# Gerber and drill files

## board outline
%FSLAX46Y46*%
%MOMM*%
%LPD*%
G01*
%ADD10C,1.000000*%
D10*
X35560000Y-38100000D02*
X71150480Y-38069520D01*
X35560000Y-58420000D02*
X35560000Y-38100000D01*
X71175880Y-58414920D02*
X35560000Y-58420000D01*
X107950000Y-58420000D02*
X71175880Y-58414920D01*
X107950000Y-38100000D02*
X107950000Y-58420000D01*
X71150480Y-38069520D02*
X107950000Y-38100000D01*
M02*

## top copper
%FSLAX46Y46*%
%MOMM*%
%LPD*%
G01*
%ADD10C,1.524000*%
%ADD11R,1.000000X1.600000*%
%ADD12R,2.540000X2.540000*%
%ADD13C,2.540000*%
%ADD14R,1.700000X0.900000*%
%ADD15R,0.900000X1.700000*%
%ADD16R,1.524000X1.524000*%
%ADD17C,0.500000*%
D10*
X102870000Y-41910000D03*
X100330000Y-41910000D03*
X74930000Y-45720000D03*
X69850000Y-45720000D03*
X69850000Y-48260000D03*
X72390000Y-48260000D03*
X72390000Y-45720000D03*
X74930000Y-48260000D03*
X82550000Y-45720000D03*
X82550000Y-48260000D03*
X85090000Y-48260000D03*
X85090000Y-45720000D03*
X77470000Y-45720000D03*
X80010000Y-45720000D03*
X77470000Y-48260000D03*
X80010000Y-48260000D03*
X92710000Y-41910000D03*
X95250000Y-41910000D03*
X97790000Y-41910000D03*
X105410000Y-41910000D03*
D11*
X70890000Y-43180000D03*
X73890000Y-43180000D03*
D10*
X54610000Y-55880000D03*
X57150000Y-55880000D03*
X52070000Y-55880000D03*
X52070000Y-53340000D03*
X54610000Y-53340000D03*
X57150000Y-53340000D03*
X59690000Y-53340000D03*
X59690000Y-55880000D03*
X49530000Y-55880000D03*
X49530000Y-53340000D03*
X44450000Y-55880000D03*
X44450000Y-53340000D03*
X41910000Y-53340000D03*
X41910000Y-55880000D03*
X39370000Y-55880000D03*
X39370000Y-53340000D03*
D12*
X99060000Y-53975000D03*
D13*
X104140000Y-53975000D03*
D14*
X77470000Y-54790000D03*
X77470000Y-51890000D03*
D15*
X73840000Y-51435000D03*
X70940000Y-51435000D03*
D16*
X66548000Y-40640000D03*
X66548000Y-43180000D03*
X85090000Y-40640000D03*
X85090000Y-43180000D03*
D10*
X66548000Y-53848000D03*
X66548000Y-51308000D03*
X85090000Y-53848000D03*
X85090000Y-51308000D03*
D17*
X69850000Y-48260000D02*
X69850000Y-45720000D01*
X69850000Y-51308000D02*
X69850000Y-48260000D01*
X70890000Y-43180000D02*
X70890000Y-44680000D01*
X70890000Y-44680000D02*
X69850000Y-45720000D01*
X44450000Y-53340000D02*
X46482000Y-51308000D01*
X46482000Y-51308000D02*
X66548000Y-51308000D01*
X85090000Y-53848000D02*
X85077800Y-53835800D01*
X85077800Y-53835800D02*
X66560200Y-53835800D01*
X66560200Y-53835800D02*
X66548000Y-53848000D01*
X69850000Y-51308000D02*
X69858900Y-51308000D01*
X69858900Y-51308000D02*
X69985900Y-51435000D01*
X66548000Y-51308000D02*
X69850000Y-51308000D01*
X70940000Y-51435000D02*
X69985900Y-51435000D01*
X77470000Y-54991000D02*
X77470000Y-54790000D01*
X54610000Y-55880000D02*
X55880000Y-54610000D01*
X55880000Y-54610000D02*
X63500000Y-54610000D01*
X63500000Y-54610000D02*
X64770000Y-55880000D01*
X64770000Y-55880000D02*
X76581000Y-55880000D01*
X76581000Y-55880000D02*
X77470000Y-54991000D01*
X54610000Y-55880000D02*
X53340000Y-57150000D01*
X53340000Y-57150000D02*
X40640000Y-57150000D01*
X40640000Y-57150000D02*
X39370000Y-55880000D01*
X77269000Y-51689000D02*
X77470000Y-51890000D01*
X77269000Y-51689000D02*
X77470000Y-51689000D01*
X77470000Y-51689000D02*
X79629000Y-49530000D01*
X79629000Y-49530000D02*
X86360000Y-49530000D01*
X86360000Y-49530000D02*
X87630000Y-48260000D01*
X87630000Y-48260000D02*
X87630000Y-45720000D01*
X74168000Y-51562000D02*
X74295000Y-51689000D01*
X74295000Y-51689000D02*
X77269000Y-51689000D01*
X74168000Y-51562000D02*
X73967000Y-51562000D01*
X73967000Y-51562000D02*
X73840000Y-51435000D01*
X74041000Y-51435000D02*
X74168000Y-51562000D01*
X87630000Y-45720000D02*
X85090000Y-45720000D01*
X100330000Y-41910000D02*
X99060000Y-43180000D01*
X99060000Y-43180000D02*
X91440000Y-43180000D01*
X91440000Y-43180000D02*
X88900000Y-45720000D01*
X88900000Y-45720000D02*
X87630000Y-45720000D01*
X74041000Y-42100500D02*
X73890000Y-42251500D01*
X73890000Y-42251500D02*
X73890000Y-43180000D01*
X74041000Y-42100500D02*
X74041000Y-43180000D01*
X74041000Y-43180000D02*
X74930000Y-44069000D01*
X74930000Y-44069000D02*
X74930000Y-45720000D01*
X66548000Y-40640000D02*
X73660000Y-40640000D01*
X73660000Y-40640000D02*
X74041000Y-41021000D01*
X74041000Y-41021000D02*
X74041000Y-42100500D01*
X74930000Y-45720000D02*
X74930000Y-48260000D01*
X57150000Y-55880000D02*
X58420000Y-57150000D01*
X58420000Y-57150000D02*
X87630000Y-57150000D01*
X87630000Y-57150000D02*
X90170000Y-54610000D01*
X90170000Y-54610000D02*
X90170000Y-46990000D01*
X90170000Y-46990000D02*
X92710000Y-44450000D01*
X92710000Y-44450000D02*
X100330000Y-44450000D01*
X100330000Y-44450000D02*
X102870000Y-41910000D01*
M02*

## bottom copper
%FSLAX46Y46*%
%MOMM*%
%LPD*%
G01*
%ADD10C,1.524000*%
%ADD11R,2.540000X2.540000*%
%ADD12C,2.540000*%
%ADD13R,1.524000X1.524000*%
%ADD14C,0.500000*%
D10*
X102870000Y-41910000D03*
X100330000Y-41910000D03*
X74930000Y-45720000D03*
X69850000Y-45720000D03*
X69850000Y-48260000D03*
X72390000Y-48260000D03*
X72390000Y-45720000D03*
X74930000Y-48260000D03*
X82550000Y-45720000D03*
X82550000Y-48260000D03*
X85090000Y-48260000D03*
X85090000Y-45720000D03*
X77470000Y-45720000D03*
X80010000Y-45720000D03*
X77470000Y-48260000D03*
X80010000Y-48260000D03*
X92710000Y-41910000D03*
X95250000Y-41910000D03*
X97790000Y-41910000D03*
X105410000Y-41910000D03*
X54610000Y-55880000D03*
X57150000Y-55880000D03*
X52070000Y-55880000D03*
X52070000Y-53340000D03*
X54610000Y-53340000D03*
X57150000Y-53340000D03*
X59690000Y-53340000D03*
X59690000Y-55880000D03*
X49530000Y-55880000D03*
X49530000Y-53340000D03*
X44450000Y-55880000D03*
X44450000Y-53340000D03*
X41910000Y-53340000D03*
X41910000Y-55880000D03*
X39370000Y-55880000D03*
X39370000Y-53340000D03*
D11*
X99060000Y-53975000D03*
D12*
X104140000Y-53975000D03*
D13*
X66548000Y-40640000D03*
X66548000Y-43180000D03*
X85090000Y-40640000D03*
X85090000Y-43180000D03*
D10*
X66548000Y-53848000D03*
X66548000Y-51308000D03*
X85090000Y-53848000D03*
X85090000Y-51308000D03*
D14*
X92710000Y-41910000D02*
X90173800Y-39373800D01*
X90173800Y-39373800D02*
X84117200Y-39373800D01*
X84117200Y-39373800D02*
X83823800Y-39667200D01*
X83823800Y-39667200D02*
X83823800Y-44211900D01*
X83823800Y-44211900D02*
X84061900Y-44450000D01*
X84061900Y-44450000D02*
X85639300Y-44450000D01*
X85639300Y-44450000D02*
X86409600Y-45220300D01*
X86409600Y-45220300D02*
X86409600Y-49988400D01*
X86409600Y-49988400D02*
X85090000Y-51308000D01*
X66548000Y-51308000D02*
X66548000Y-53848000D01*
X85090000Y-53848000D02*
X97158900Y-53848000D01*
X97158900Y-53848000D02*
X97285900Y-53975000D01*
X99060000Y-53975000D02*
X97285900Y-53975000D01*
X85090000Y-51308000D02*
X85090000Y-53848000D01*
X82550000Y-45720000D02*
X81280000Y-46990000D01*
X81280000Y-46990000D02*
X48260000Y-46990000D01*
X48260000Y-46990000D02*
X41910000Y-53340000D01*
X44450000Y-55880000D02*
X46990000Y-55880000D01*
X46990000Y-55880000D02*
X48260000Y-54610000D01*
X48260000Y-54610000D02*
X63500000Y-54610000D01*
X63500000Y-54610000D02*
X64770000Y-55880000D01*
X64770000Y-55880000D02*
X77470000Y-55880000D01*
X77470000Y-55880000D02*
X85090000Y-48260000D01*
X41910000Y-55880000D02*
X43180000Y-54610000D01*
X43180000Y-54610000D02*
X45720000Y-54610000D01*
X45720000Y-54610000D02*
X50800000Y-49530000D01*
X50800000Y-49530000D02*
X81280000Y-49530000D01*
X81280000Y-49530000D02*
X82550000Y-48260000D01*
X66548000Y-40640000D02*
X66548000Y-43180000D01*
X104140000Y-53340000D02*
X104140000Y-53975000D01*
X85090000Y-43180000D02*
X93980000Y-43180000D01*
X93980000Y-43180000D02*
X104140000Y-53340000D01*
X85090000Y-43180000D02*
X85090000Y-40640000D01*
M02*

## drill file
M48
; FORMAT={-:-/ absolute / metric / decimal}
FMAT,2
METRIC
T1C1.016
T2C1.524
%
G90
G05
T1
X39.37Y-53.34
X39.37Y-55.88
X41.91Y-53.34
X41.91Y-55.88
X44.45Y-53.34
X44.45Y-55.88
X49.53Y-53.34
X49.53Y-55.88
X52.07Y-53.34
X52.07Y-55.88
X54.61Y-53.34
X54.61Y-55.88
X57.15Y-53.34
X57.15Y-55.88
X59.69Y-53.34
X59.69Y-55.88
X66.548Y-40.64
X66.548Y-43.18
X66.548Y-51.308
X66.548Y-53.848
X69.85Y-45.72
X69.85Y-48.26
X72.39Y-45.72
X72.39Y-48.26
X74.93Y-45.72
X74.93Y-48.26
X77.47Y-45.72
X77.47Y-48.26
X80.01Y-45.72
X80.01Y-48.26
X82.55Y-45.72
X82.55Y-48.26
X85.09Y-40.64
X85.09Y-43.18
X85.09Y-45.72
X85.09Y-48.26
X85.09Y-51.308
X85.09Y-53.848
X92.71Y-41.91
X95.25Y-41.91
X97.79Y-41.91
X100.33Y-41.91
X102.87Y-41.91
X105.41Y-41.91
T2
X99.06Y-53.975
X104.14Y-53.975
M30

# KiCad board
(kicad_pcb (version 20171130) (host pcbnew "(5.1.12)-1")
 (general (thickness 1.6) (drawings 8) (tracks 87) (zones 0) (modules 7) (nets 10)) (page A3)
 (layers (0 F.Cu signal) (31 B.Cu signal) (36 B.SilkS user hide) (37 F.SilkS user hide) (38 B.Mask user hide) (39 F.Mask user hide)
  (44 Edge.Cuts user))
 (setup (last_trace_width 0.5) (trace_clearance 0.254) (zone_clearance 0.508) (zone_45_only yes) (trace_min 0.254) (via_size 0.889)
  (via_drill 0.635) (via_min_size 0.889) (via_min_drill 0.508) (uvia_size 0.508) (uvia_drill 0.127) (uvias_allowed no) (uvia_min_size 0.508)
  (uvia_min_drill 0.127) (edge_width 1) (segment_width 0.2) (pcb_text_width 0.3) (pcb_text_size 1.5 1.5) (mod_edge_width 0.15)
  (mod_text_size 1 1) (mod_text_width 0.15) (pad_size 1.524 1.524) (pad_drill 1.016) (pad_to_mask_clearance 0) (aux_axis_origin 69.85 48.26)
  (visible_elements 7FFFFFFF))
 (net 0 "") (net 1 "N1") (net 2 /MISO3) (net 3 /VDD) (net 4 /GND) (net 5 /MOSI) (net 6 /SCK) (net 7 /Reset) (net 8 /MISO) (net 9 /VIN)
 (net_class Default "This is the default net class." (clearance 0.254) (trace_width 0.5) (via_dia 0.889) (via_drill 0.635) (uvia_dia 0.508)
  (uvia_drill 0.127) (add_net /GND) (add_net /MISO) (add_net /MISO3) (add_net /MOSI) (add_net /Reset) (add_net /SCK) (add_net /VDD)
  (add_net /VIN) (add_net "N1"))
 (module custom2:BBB (layer B.Cu) (at 97.79 45.72 180)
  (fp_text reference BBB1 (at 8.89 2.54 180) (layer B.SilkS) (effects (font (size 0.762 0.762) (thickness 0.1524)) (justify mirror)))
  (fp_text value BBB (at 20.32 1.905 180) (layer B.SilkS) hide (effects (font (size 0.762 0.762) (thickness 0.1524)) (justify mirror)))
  (pad TxD thru_hole circle (at -5.08 3.81) (size 1.524 1.524) (drill 1.016) (layers *.Cu *.Mask) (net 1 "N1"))
  (pad RxD thru_hole circle (at -2.54 3.81) (size 1.524 1.524) (drill 1.016) (layers *.Cu *.Mask) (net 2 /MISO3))
  (pad VDD thru_hole circle (at 22.86 0) (size 1.524 1.524) (drill 1.016) (layers *.Cu *.Mask) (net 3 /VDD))
  (pad GND thru_hole circle (at 27.94 0) (size 1.524 1.524) (drill 1.016) (layers *.Cu *.Mask) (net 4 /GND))
  (pad GND thru_hole circle (at 27.94 -2.54) (size 1.524 1.524) (drill 1.016) (layers *.Cu *.Mask) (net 4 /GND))
  (pad X thru_hole circle (at 25.4 -2.54) (size 1.524 1.524) (drill 1.016) (layers *.Cu *.Mask))
  (pad X thru_hole circle (at 25.4 0) (size 1.524 1.524) (drill 1.016) (layers *.Cu *.Mask))
  (pad VDD thru_hole circle (at 22.86 -2.54) (size 1.524 1.524) (drill 1.016) (layers *.Cu *.Mask) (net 3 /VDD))
  (pad 60 thru_hole circle (at 15.24 0) (size 1.524 1.524) (drill 1.016) (layers *.Cu *.Mask B.SilkS) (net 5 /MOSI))
  (pad 30 thru_hole circle (at 15.24 -2.54) (size 1.524 1.524) (drill 1.016) (layers *.Cu *.Mask B.SilkS) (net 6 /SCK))
  (pad 31 thru_hole circle (at 12.7 -2.54) (size 1.524 1.524) (drill 1.016) (layers *.Cu *.Mask B.SilkS) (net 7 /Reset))
  (pad 50 thru_hole circle (at 12.7 0) (size 1.524 1.524) (drill 1.016) (layers *.Cu *.Mask B.SilkS) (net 2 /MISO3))
  (pad VSYS thru_hole circle (at 20.32 0) (size 1.524 1.524) (drill 1.016) (layers *.Cu *.Mask B.SilkS))
  (pad RST thru_hole circle (at 17.78 0) (size 1.524 1.524) (drill 1.016) (layers *.Cu *.Mask B.SilkS))
  (pad VSYS thru_hole circle (at 20.32 -2.54) (size 1.524 1.524) (drill 1.016) (layers *.Cu *.Mask B.SilkS))
  (pad PBUT thru_hole circle (at 17.78 -2.54) (size 1.524 1.524) (drill 1.016) (layers *.Cu *.Mask B.SilkS))
  (pad GND thru_hole circle (at 5.08 3.81) (size 1.524 1.524) (drill 1.016) (layers *.Cu *.Mask B.SilkS) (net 4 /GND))
  (pad X thru_hole circle (at 2.54 3.81) (size 1.524 1.524) (drill 1.016) (layers *.Cu *.Mask B.SilkS))
  (pad X thru_hole circle (at 0 3.81) (size 1.524 1.524) (drill 1.016) (layers *.Cu *.Mask B.SilkS))
  (pad X thru_hole circle (at -7.62 3.81) (size 1.524 1.524) (drill 1.016) (layers *.Cu *.Mask B.SilkS)))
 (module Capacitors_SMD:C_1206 (layer F.Cu) (at 72.39 43.18)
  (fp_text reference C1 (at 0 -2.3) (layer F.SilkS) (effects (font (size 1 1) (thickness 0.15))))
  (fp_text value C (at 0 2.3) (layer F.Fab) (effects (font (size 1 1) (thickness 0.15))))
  (pad 1 smd rect (at -1.5 0) (size 1 1.6) (layers F.Cu F.Mask) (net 4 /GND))
  (pad 2 smd rect (at 1.5 0) (size 1 1.6) (layers F.Cu F.Mask) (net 3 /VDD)))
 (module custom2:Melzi (layer B.Cu) (at 43.18 55.88 180)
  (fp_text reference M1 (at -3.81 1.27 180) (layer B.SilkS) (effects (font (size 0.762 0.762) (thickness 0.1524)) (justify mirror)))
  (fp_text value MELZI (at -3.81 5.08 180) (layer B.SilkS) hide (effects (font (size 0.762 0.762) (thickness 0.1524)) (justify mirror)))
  (pad TxD thru_hole circle (at -11.43 0) (size 1.524 1.524) (drill 1.016) (layers *.Cu *.Mask) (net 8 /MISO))
  (pad RxD thru_hole circle (at -13.97 0) (size 1.524 1.524) (drill 1.016) (layers *.Cu *.Mask) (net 1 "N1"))
  (pad D16 thru_hole circle (at -8.89 0) (size 1.524 1.524) (drill 1.016) (layers *.Cu *.Mask B.SilkS))
  (pad A2 thru_hole circle (at -8.89 2.54) (size 1.524 1.524) (drill 1.016) (layers *.Cu *.Mask B.SilkS))
  (pad A3 thru_hole circle (at -11.43 2.54) (size 1.524 1.524) (drill 1.016) (layers *.Cu *.Mask B.SilkS))
  (pad A4 thru_hole circle (at -13.97 2.54) (size 1.524 1.524) (drill 1.016) (layers *.Cu *.Mask B.SilkS))
  (pad GND2 thru_hole circle (at -16.51 2.54) (size 1.524 1.524) (drill 1.016) (layers *.Cu *.Mask B.SilkS))
  (pad 5V thru_hole circle (at -16.51 0) (size 1.524 1.524) (drill 1.016) (layers *.Cu *.Mask B.SilkS))
  (pad D17 thru_hole circle (at -6.35 0) (size 1.524 1.524) (drill 1.016) (layers *.Cu *.Mask B.SilkS))
  (pad A1 thru_hole circle (at -6.35 2.54) (size 1.524 1.524) (drill 1.016) (layers *.Cu *.Mask B.SilkS))
  (pad ~RST thru_hole circle (at -1.27 0) (size 1.524 1.524) (drill 1.016) (layers *.Cu *.Mask B.SilkS) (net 7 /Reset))
  (pad GND thru_hole circle (at -1.27 2.54) (size 1.524 1.524) (drill 1.016) (layers *.Cu *.Mask B.SilkS) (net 4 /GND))
  (pad MOSI thru_hole circle (at 1.27 2.54) (size 1.524 1.524) (drill 1.016) (layers *.Cu *.Mask B.SilkS) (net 5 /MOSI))
  (pad SCK thru_hole circle (at 1.27 0) (size 1.524 1.524) (drill 1.016) (layers *.Cu *.Mask B.SilkS) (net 6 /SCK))
  (pad MISO thru_hole circle (at 3.81 0) (size 1.524 1.524) (drill 1.016) (layers *.Cu *.Mask B.SilkS) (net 8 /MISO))
  (pad 5V thru_hole circle (at 3.81 2.54) (size 1.524 1.524) (drill 1.016) (layers *.Cu *.Mask B.SilkS)))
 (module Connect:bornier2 (layer B.Cu) (at 101.6 53.975)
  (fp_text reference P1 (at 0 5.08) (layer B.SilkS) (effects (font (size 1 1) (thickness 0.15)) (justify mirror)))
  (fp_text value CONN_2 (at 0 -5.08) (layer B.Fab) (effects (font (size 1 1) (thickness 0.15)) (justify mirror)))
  (pad 1 thru_hole rect (at -2.54 0) (size 2.54 2.54) (drill 1.524) (layers *.Cu *.Mask B.SilkS) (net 4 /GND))
  (pad 2 thru_hole circle (at 2.54 0) (size 2.54 2.54) (drill 1.524) (layers *.Cu *.Mask B.SilkS) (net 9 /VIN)))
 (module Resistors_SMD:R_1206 (layer F.Cu) (at 77.47 53.34 90)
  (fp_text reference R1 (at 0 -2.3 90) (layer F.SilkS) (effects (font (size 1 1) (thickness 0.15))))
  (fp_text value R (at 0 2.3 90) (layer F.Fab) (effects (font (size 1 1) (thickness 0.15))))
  (pad 1 smd rect (at -1.45 0 90) (size 0.9 1.7) (layers F.Cu F.Mask) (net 8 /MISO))
  (pad 2 smd rect (at 1.45 0 90) (size 0.9 1.7) (layers F.Cu F.Mask) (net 2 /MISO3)))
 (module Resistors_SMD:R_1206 (layer F.Cu) (at 72.39 51.435 180)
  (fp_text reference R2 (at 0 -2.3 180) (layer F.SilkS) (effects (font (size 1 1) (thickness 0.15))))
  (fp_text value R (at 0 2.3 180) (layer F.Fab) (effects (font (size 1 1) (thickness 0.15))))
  (pad 1 smd rect (at -1.45 0 180) (size 0.9 1.7) (layers F.Cu F.Mask) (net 2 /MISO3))
  (pad 2 smd rect (at 1.45 0 180) (size 0.9 1.7) (layers F.Cu F.Mask) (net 4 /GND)))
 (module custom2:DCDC (layer B.Cu) (at 66.04 40.64)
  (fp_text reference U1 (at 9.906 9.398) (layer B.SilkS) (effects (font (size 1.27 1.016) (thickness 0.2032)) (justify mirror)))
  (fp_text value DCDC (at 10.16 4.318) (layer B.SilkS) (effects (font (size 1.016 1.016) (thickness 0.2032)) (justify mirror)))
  (pad Vout thru_hole rect (at 0.508 0 270) (size 1.524 1.524) (drill 1.016) (layers *.Cu *.Mask B.SilkS) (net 3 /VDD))
  (pad Vout thru_hole rect (at 0.508 2.54 270) (size 1.524 1.524) (drill 1.016) (layers *.Cu *.Mask B.SilkS) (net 3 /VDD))
  (pad Vin thru_hole rect (at 19.05 0 270) (size 1.524 1.524) (drill 1.016) (layers *.Cu *.Mask B.SilkS) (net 9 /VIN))
  (pad Vin thru_hole rect (at 19.05 2.54 270) (size 1.524 1.524) (drill 1.016) (layers *.Cu *.Mask B.SilkS) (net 9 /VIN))
  (pad GND2 thru_hole circle (at 0.508 13.208 270) (size 1.524 1.524) (drill 1.016) (layers *.Cu *.Mask B.SilkS) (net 4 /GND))
  (pad GND2 thru_hole circle (at 0.508 10.668 270) (size 1.524 1.524) (drill 1.016) (layers *.Cu *.Mask B.SilkS) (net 4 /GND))
  (pad GND thru_hole circle (at 19.05 13.208 270) (size 1.524 1.524) (drill 1.016) (layers *.Cu *.Mask B.SilkS) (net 4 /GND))
  (pad GND thru_hole circle (at 19.05 10.668 270) (size 1.524 1.524) (drill 1.016) (layers *.Cu *.Mask B.SilkS) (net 4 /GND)))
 (gr_line (start 35.56 38.1) (end 71.15048 38.06952) (angle 90) (layer Edge.Cuts) (width 1))
 (gr_line (start 35.56 58.42) (end 35.56 38.1) (angle 90) (layer Edge.Cuts) (width 1))
 (gr_line (start 71.17588 58.41492) (end 35.56 58.42) (angle 90) (layer Edge.Cuts) (width 1))
 (gr_line (start 107.95 58.42) (end 71.17588 58.41492) (angle 90) (layer Edge.Cuts) (width 1))
 (gr_line (start 107.95 38.1) (end 107.95 58.42) (angle 90) (layer Edge.Cuts) (width 1))
 (gr_line (start 71.15048 38.06952) (end 107.95 38.1) (angle 90) (layer Edge.Cuts) (width 1))
 (segment (start 69.85 48.26) (end 69.85 45.72) (width 0.5) (layer F.Cu) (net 4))
 (segment (start 69.85 51.308) (end 69.85 48.26) (width 0.5) (layer F.Cu) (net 4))
 (segment (start 92.71 41.91) (end 90.1738 39.3738) (width 0.5) (layer B.Cu) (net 4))
 (segment (start 90.1738 39.3738) (end 84.1172 39.3738) (width 0.5) (layer B.Cu) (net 4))
 (segment (start 84.1172 39.3738) (end 83.8238 39.6672) (width 0.5) (layer B.Cu) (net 4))
 (segment (start 83.8238 39.6672) (end 83.8238 44.2119) (width 0.5) (layer B.Cu) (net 4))
 (segment (start 83.8238 44.2119) (end 84.0619 44.45) (width 0.5) (layer B.Cu) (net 4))
 (segment (start 84.0619 44.45) (end 85.6393 44.45) (width 0.5) (layer B.Cu) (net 4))
 (segment (start 85.6393 44.45) (end 86.4096 45.2203) (width 0.5) (layer B.Cu) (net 4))
 (segment (start 86.4096 45.2203) (end 86.4096 49.9884) (width 0.5) (layer B.Cu) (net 4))
 (segment (start 86.4096 49.9884) (end 85.09 51.308) (width 0.5) (layer B.Cu) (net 4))
 (segment (start 70.89 43.18) (end 70.89 44.68) (width 0.5) (layer F.Cu) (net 4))
 (segment (start 70.89 44.68) (end 69.85 45.72) (width 0.5) (layer F.Cu) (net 4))
 (segment (start 44.45 53.34) (end 46.482 51.308) (width 0.5) (layer F.Cu) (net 4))
 (segment (start 46.482 51.308) (end 66.548 51.308) (width 0.5) (layer F.Cu) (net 4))
 (segment (start 85.09 53.848) (end 85.0778 53.8358) (width 0.5) (layer F.Cu) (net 4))
 (segment (start 85.0778 53.8358) (end 66.5602 53.8358) (width 0.5) (layer F.Cu) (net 4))
 (segment (start 66.5602 53.8358) (end 66.548 53.848) (width 0.5) (layer F.Cu) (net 4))
 (segment (start 69.85 51.308) (end 69.8589 51.308) (width 0.5) (layer F.Cu) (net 4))
 (segment (start 69.8589 51.308) (end 69.9859 51.435) (width 0.5) (layer F.Cu) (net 4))
 (segment (start 66.548 51.308) (end 69.85 51.308) (width 0.5) (layer F.Cu) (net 4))
 (segment (start 70.94 51.435) (end 69.9859 51.435) (width 0.5) (layer F.Cu) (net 4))
 (segment (start 66.548 51.308) (end 66.548 53.848) (width 0.5) (layer B.Cu) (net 4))
 (segment (start 85.09 53.848) (end 97.1589 53.848) (width 0.5) (layer B.Cu) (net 4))
 (segment (start 97.1589 53.848) (end 97.2859 53.975) (width 0.5) (layer B.Cu) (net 4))
 (segment (start 99.06 53.975) (end 97.2859 53.975) (width 0.5) (layer B.Cu) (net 4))
 (segment (start 85.09 51.308) (end 85.09 53.848) (width 0.5) (layer B.Cu) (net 4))
 (segment (start 77.47 54.991) (end 77.47 54.79) (width 0.5) (layer F.Cu) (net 8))
 (segment (start 54.61 55.88) (end 55.88 54.61) (width 0.5) (layer F.Cu) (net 8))
 (segment (start 55.88 54.61) (end 63.5 54.61) (width 0.5) (layer F.Cu) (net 8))
 (segment (start 63.5 54.61) (end 64.77 55.88) (width 0.5) (layer F.Cu) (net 8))
 (segment (start 64.77 55.88) (end 76.581 55.88) (width 0.5) (layer F.Cu) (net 8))
 (segment (start 76.581 55.88) (end 77.47 54.991) (width 0.5) (layer F.Cu) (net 8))
 (segment (start 54.61 55.88) (end 53.34 57.15) (width 0.5) (layer F.Cu) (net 8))
 (segment (start 53.34 57.15) (end 40.64 57.15) (width 0.5) (layer F.Cu) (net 8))
 (segment (start 40.64 57.15) (end 39.37 55.88) (width 0.5) (layer F.Cu) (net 8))
 (segment (start 77.269 51.689) (end 77.47 51.89) (width 0.5) (layer F.Cu) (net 2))
 (segment (start 77.269 51.689) (end 77.47 51.689) (width 0.5) (layer F.Cu) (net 2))
 (segment (start 77.47 51.689) (end 79.629 49.53) (width 0.5) (layer F.Cu) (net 2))
 (segment (start 79.629 49.53) (end 86.36 49.53) (width 0.5) (layer F.Cu) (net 2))
 (segment (start 86.36 49.53) (end 87.63 48.26) (width 0.5) (layer F.Cu) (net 2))
 (segment (start 87.63 48.26) (end 87.63 45.72) (width 0.5) (layer F.Cu) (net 2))
 (segment (start 74.168 51.562) (end 74.295 51.689) (width 0.5) (layer F.Cu) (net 2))
 (segment (start 74.295 51.689) (end 77.269 51.689) (width 0.5) (layer F.Cu) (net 2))
 (segment (start 74.168 51.562) (end 73.967 51.562) (width 0.5) (layer F.Cu) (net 2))
 (segment (start 73.967 51.562) (end 73.84 51.435) (width 0.5) (layer F.Cu) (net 2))
 (segment (start 74.041 51.435) (end 74.168 51.562) (width 0.5) (layer F.Cu) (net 2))
 (segment (start 87.63 45.72) (end 85.09 45.72) (width 0.5) (layer F.Cu) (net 2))
 (segment (start 100.33 41.91) (end 99.06 43.18) (width 0.5) (layer F.Cu) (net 2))
 (segment (start 99.06 43.18) (end 91.44 43.18) (width 0.5) (layer F.Cu) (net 2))
 (segment (start 91.44 43.18) (end 88.9 45.72) (width 0.5) (layer F.Cu) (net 2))
 (segment (start 88.9 45.72) (end 87.63 45.72) (width 0.5) (layer F.Cu) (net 2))
 (segment (start 82.55 45.72) (end 81.28 46.99) (width 0.5) (layer B.Cu) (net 5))
 (segment (start 81.28 46.99) (end 48.26 46.99) (width 0.5) (layer B.Cu) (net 5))
 (segment (start 48.26 46.99) (end 41.91 53.34) (width 0.5) (layer B.Cu) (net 5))
 (segment (start 44.45 55.88) (end 46.99 55.88) (width 0.5) (layer B.Cu) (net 7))
 (segment (start 46.99 55.88) (end 48.26 54.61) (width 0.5) (layer B.Cu) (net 7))
 (segment (start 48.26 54.61) (end 63.5 54.61) (width 0.5) (layer B.Cu) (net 7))
 (segment (start 63.5 54.61) (end 64.77 55.88) (width 0.5) (layer B.Cu) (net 7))
 (segment (start 64.77 55.88) (end 77.47 55.88) (width 0.5) (layer B.Cu) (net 7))
 (segment (start 77.47 55.88) (end 85.09 48.26) (width 0.5) (layer B.Cu) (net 7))
 (segment (start 41.91 55.88) (end 43.18 54.61) (width 0.5) (layer B.Cu) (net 6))
 (segment (start 43.18 54.61) (end 45.72 54.61) (width 0.5) (layer B.Cu) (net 6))
 (segment (start 45.72 54.61) (end 50.8 49.53) (width 0.5) (layer B.Cu) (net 6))
 (segment (start 50.8 49.53) (end 81.28 49.53) (width 0.5) (layer B.Cu) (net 6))
 (segment (start 81.28 49.53) (end 82.55 48.26) (width 0.5) (layer B.Cu) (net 6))
 (segment (start 74.041 42.1005) (end 73.89 42.2515) (width 0.5) (layer F.Cu) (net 3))
 (segment (start 73.89 42.2515) (end 73.89 43.18) (width 0.5) (layer F.Cu) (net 3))
 (segment (start 74.041 42.1005) (end 74.041 43.18) (width 0.5) (layer F.Cu) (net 3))
 (segment (start 74.041 43.18) (end 74.93 44.069) (width 0.5) (layer F.Cu) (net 3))
 (segment (start 74.93 44.069) (end 74.93 45.72) (width 0.5) (layer F.Cu) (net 3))
 (segment (start 66.548 40.64) (end 73.66 40.64) (width 0.5) (layer F.Cu) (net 3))
 (segment (start 73.66 40.64) (end 74.041 41.021) (width 0.5) (layer F.Cu) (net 3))
 (segment (start 74.041 41.021) (end 74.041 42.1005) (width 0.5) (layer F.Cu) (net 3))
 (segment (start 66.548 40.64) (end 66.548 43.18) (width 0.5) (layer B.Cu) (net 3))
 (segment (start 74.93 45.72) (end 74.93 48.26) (width 0.5) (layer F.Cu) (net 3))
 (segment (start 104.14 53.34) (end 104.14 53.975) (width 0.5) (layer B.Cu) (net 9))
 (segment (start 85.09 43.18) (end 93.98 43.18) (width 0.5) (layer B.Cu) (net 9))
 (segment (start 93.98 43.18) (end 104.14 53.34) (width 0.5) (layer B.Cu) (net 9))
 (segment (start 85.09 43.18) (end 85.09 40.64) (width 0.5) (layer B.Cu) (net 9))
 (segment (start 57.15 55.88) (end 58.42 57.15) (width 0.5) (layer F.Cu) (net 1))
 (segment (start 58.42 57.15) (end 87.63 57.15) (width 0.5) (layer F.Cu) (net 1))
 (segment (start 87.63 57.15) (end 90.17 54.61) (width 0.5) (layer F.Cu) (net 1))
 (segment (start 90.17 54.61) (end 90.17 46.99) (width 0.5) (layer F.Cu) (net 1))
 (segment (start 90.17 46.99) (end 92.71 44.45) (width 0.5) (layer F.Cu) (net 1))
 (segment (start 92.71 44.45) (end 100.33 44.45) (width 0.5) (layer F.Cu) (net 1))
 (segment (start 100.33 44.45) (end 102.87 41.91) (width 0.5) (layer F.Cu) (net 1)))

